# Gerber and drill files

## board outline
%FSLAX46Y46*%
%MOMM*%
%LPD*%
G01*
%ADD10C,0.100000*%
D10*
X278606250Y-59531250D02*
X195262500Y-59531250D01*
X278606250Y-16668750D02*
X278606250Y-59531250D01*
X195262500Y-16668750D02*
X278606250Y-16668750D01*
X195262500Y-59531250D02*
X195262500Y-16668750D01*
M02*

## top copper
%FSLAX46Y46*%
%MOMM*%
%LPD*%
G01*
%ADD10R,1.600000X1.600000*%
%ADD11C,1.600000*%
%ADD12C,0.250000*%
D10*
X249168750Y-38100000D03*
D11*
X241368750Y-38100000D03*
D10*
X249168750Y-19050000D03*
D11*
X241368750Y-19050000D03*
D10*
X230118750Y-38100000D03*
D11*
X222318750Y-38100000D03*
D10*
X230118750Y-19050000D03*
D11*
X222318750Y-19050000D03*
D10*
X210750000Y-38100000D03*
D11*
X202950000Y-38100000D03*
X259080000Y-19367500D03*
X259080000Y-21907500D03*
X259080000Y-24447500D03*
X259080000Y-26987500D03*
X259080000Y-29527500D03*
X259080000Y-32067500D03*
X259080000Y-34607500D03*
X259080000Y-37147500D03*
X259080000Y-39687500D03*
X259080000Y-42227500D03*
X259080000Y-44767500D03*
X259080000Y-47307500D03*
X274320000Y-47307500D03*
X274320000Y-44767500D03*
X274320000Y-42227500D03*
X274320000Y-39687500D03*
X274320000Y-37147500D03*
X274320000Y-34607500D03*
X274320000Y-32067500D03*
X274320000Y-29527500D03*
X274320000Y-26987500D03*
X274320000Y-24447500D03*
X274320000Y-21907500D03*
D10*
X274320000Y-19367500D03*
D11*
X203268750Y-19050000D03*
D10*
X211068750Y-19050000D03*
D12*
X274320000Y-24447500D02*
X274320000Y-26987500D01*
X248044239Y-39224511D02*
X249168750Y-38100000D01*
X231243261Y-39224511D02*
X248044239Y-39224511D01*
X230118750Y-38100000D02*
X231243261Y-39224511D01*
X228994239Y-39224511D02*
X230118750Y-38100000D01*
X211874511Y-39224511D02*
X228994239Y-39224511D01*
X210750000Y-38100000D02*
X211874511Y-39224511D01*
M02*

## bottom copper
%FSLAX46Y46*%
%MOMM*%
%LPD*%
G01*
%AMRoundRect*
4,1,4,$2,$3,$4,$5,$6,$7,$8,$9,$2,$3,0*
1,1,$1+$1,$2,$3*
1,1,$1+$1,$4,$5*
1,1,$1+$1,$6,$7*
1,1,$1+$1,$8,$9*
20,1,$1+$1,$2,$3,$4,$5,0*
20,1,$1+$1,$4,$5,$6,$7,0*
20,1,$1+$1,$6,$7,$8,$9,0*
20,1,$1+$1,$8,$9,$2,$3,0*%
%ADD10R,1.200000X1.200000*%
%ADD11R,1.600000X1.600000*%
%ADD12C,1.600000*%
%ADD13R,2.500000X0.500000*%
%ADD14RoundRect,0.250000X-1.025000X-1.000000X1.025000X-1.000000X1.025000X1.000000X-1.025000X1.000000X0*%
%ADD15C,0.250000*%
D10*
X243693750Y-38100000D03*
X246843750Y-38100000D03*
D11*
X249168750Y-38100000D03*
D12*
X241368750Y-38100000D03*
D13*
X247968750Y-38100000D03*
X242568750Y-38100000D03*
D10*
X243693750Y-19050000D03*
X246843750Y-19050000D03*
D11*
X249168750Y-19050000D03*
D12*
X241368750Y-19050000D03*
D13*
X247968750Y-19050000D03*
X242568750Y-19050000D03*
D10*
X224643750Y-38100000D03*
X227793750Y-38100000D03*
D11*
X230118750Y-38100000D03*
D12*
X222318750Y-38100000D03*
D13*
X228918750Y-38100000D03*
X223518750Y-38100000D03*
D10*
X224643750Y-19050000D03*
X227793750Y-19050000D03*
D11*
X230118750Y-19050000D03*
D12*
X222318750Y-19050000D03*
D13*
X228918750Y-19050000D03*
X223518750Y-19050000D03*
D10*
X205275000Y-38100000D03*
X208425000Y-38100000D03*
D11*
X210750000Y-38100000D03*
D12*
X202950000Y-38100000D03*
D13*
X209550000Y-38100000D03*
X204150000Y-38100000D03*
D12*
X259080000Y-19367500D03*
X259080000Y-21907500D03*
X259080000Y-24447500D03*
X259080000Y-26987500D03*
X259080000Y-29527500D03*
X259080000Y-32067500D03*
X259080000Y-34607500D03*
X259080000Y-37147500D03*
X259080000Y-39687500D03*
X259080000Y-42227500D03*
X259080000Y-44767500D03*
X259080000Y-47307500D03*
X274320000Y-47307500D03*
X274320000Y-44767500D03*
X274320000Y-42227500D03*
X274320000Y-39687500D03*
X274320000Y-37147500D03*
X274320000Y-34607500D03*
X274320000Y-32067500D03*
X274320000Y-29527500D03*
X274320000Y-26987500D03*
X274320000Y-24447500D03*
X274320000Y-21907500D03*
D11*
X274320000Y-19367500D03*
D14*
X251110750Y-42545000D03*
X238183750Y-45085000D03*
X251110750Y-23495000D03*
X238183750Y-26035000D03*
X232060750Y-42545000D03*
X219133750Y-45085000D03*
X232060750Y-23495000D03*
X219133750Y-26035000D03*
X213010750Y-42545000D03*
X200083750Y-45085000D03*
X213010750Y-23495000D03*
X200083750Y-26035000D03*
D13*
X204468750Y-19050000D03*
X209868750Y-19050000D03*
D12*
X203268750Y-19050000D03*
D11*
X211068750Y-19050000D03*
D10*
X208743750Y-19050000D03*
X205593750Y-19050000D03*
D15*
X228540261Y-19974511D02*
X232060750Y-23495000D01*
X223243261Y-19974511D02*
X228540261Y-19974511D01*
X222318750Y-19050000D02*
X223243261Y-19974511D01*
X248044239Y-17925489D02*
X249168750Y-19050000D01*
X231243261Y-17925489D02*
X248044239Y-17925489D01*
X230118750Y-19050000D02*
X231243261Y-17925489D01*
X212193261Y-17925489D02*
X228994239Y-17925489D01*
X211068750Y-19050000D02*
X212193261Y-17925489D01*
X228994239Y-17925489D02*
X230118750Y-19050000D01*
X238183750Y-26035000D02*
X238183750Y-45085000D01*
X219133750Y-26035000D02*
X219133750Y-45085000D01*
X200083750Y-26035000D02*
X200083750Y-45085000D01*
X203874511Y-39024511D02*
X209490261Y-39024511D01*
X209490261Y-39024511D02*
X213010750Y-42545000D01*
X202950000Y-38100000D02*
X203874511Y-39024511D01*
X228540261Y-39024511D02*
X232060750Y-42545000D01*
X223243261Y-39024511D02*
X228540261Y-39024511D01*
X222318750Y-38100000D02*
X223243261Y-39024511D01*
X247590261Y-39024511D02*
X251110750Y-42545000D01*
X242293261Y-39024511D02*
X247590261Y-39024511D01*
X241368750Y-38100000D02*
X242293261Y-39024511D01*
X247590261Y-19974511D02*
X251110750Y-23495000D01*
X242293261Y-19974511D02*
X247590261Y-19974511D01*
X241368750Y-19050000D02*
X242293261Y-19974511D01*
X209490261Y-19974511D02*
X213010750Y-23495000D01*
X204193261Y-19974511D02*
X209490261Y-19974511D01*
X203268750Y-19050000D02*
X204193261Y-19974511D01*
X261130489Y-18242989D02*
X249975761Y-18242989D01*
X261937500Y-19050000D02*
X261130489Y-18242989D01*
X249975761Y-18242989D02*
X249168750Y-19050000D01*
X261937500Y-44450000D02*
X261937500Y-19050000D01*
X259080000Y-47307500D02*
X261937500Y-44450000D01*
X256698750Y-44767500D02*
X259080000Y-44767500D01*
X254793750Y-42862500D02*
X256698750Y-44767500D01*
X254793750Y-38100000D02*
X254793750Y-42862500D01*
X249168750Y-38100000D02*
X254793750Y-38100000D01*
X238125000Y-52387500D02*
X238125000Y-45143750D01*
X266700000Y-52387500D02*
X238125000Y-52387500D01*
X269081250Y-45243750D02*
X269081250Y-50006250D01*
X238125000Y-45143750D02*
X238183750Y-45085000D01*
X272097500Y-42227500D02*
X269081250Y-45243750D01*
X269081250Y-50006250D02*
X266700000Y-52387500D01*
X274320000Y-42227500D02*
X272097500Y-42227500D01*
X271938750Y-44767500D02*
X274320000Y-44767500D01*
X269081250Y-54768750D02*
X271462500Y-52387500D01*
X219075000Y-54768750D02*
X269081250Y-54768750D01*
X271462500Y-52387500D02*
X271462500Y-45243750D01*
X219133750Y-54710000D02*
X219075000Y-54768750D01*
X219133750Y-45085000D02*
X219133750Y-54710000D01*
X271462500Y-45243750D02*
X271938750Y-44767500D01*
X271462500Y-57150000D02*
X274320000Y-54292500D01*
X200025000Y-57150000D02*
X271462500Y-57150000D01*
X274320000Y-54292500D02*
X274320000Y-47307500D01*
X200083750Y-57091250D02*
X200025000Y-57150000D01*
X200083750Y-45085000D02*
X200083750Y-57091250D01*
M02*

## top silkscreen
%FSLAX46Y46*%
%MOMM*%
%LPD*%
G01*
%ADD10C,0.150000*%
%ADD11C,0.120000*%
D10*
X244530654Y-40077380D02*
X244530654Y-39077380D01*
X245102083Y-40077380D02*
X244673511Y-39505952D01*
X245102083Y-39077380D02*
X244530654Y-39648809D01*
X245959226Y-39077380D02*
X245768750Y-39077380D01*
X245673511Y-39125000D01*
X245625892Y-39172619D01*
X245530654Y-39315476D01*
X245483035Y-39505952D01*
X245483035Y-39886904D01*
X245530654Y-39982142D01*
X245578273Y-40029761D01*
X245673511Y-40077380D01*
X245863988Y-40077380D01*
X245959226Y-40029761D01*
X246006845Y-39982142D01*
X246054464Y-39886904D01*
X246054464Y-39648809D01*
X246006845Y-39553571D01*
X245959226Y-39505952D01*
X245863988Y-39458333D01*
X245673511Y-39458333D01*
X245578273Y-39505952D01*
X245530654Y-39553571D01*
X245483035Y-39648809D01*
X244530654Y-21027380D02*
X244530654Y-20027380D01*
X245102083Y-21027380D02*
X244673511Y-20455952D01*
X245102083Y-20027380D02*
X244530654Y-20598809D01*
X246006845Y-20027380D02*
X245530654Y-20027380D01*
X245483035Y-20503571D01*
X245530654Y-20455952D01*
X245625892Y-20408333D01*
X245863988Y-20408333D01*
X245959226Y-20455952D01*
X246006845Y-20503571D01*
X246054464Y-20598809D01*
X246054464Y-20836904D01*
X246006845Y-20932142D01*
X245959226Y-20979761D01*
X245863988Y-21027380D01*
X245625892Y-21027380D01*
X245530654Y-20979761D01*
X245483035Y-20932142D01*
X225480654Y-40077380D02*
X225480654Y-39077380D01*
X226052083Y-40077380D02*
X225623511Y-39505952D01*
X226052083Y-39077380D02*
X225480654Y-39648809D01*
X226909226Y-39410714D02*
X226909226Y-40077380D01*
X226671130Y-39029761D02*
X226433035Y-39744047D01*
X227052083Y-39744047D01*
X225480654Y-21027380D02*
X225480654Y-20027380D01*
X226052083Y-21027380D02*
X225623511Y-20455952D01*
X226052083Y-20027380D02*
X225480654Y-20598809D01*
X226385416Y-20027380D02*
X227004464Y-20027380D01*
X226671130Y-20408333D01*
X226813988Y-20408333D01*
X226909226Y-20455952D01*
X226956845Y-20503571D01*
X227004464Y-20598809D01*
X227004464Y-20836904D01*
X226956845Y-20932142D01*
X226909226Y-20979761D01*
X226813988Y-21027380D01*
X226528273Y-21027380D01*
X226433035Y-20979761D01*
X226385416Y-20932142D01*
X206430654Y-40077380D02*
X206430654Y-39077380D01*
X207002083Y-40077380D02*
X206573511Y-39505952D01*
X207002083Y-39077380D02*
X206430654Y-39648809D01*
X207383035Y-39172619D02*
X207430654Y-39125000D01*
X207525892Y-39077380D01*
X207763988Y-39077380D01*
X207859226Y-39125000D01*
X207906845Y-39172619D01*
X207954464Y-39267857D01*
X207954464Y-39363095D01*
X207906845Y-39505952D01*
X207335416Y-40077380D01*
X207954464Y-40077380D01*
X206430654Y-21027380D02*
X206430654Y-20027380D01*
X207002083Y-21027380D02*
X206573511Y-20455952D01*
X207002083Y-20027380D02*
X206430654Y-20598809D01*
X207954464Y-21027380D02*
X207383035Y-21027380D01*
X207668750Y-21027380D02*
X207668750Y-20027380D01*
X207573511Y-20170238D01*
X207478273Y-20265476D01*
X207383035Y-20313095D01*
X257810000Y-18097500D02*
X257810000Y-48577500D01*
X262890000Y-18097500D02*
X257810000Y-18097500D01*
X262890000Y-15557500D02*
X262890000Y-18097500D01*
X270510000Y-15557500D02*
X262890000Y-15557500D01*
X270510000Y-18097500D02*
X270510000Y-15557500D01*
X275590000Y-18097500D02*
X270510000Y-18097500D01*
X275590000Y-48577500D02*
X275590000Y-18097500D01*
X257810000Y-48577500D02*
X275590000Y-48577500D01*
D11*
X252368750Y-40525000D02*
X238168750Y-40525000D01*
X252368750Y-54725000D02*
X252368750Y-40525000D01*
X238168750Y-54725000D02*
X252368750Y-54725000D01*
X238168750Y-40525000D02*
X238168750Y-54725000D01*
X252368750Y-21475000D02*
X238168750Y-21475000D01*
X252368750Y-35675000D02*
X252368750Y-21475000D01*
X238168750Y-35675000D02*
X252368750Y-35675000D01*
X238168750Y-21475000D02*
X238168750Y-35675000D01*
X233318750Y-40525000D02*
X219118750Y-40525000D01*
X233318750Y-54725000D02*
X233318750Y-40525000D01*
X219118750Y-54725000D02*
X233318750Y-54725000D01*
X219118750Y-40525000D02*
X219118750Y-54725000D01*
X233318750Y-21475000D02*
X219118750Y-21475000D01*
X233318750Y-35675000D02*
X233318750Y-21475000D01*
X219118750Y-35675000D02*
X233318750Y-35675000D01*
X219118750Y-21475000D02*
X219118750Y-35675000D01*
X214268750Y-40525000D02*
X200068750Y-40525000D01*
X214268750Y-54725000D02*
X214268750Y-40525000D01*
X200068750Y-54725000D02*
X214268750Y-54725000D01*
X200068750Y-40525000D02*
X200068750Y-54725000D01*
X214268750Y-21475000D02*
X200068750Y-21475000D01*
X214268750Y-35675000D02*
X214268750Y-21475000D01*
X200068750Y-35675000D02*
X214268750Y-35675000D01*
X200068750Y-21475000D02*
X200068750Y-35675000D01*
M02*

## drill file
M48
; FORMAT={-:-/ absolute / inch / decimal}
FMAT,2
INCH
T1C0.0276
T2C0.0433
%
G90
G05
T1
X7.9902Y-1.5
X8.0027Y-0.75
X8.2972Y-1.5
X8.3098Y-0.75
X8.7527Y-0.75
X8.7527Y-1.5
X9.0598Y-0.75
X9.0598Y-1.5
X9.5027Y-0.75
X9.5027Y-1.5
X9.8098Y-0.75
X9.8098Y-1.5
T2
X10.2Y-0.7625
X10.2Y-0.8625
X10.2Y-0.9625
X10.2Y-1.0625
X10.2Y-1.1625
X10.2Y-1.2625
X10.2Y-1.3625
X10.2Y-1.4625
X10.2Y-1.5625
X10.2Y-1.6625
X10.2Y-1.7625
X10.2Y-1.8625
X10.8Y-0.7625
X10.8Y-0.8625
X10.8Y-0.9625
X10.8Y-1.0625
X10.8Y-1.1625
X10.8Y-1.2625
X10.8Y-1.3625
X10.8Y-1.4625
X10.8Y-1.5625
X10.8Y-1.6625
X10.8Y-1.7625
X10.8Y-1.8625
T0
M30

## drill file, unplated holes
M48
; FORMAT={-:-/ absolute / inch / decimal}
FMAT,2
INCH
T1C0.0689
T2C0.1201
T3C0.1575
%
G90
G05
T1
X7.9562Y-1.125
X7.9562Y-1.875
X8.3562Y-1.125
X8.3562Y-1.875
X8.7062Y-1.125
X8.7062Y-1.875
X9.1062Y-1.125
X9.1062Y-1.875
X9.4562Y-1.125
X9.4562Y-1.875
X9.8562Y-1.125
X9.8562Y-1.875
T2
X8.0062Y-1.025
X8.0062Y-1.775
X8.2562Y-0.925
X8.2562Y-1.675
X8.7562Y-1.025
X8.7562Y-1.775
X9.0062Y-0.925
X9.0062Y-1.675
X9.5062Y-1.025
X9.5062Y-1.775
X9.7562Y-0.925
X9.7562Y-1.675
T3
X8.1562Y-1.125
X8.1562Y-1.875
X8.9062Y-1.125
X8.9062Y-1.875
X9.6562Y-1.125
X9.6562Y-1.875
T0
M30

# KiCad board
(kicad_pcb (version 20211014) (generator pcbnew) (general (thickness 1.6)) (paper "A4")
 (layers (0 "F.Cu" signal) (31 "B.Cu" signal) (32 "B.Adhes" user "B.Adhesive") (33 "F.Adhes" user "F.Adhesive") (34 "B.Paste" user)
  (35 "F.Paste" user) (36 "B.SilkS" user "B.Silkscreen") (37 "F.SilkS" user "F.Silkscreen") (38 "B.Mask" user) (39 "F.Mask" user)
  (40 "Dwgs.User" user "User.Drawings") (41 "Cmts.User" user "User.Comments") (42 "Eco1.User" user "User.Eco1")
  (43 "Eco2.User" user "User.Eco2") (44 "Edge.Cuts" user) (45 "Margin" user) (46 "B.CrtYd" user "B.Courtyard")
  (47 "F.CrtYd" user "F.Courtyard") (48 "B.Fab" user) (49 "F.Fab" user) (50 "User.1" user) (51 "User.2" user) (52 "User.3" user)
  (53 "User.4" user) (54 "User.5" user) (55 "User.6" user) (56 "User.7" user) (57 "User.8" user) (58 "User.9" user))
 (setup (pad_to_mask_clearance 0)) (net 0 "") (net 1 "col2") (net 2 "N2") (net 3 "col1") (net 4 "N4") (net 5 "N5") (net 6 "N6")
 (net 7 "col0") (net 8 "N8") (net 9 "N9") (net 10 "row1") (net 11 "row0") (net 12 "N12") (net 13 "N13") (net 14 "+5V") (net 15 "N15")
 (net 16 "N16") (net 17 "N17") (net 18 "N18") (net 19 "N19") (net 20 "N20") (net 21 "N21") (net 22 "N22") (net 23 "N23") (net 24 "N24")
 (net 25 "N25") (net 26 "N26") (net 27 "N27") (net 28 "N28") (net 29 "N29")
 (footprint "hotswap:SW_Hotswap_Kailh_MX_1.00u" (layer "F.Cu") (at 245.26875 28.575)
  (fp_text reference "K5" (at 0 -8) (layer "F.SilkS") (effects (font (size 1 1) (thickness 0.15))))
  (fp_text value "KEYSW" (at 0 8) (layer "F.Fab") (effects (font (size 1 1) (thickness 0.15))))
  (fp_line (start -7.1 7.1) (end 7.1 7.1) (layer "F.SilkS") (width 0.12))
  (fp_line (start -7.1 -7.1) (end -7.1 7.1) (layer "F.SilkS") (width 0.12))
  (fp_line (start 7.1 -7.1) (end -7.1 -7.1) (layer "F.SilkS") (width 0.12))
  (fp_line (start 7.1 7.1) (end 7.1 -7.1) (layer "F.SilkS") (width 0.12))
  (pad "" np_thru_hole circle locked (at 0 0) (size 4 4) (drill 4) (layers *.Cu *.Mask))
  (pad "" np_thru_hole circle locked (at 2.54 -5.08) (size 3.05 3.05) (drill 3.05) (layers *.Cu *.Mask))
  (pad "" np_thru_hole circle locked (at -3.81 -2.54) (size 3.05 3.05) (drill 3.05) (layers *.Cu *.Mask))
  (pad "" np_thru_hole circle locked (at -5.08 0) (size 1.75 1.75) (drill 1.75) (layers *.Cu *.Mask))
  (pad "" np_thru_hole circle locked (at 5.08 0) (size 1.75 1.75) (drill 1.75) (layers *.Cu *.Mask))
  (pad "1" smd roundrect locked (at -7.085 -2.54) (size 2.55 2.5) (layers "B.Cu" "B.Paste" "B.Mask") (roundrect_rratio 0.1) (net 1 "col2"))
  (pad "2" smd roundrect locked (at 5.842 -5.08) (size 2.55 2.5) (layers "B.Cu" "B.Paste" "B.Mask") (roundrect_rratio 0.1) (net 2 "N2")))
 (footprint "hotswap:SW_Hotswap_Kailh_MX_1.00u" (layer "F.Cu") (at 226.21875 47.625)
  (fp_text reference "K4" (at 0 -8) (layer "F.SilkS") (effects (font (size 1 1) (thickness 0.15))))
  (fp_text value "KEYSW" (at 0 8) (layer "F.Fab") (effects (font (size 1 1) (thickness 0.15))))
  (fp_line (start -7.1 -7.1) (end -7.1 7.1) (layer "F.SilkS") (width 0.12))
  (fp_line (start -7.1 7.1) (end 7.1 7.1) (layer "F.SilkS") (width 0.12))
  (fp_line (start 7.1 -7.1) (end -7.1 -7.1) (layer "F.SilkS") (width 0.12))
  (fp_line (start 7.1 7.1) (end 7.1 -7.1) (layer "F.SilkS") (width 0.12))
  (pad "" np_thru_hole circle locked (at 2.54 -5.08) (size 3.05 3.05) (drill 3.05) (layers *.Cu *.Mask))
  (pad "" np_thru_hole circle locked (at 5.08 0) (size 1.75 1.75) (drill 1.75) (layers *.Cu *.Mask))
  (pad "" np_thru_hole circle locked (at -5.08 0) (size 1.75 1.75) (drill 1.75) (layers *.Cu *.Mask))
  (pad "" np_thru_hole circle locked (at -3.81 -2.54) (size 3.05 3.05) (drill 3.05) (layers *.Cu *.Mask))
  (pad "" np_thru_hole circle locked (at 0 0) (size 4 4) (drill 4) (layers *.Cu *.Mask))
  (pad "1" smd roundrect locked (at -7.085 -2.54) (size 2.55 2.5) (layers "B.Cu" "B.Paste" "B.Mask") (roundrect_rratio 0.1) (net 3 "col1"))
  (pad "2" smd roundrect locked (at 5.842 -5.08) (size 2.55 2.5) (layers "B.Cu" "B.Paste" "B.Mask") (roundrect_rratio 0.1) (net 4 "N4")))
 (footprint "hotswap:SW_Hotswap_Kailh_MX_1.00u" (layer "F.Cu") (at 226.21875 28.575)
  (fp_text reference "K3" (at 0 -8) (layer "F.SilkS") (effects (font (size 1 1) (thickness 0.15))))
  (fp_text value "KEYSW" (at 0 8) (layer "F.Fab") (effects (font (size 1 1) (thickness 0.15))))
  (fp_line (start 7.1 7.1) (end 7.1 -7.1) (layer "F.SilkS") (width 0.12))
  (fp_line (start -7.1 -7.1) (end -7.1 7.1) (layer "F.SilkS") (width 0.12))
  (fp_line (start -7.1 7.1) (end 7.1 7.1) (layer "F.SilkS") (width 0.12))
  (fp_line (start 7.1 -7.1) (end -7.1 -7.1) (layer "F.SilkS") (width 0.12))
  (pad "" np_thru_hole circle locked (at 5.08 0) (size 1.75 1.75) (drill 1.75) (layers *.Cu *.Mask))
  (pad "" np_thru_hole circle locked (at -5.08 0) (size 1.75 1.75) (drill 1.75) (layers *.Cu *.Mask))
  (pad "" np_thru_hole circle locked (at 0 0) (size 4 4) (drill 4) (layers *.Cu *.Mask))
  (pad "" np_thru_hole circle locked (at -3.81 -2.54) (size 3.05 3.05) (drill 3.05) (layers *.Cu *.Mask))
  (pad "" np_thru_hole circle locked (at 2.54 -5.08) (size 3.05 3.05) (drill 3.05) (layers *.Cu *.Mask))
  (pad "1" smd roundrect locked (at -7.085 -2.54) (size 2.55 2.5) (layers "B.Cu" "B.Paste" "B.Mask") (roundrect_rratio 0.1) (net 3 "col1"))
  (pad "2" smd roundrect locked (at 5.842 -5.08) (size 2.55 2.5) (layers "B.Cu" "B.Paste" "B.Mask") (roundrect_rratio 0.1) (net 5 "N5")))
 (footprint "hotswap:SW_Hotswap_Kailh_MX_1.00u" (layer "F.Cu") (at 245.26875 47.625)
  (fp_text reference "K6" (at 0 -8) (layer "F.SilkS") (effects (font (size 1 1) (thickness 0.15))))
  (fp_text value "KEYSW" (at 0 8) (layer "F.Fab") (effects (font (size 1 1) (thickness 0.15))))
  (fp_line (start -7.1 -7.1) (end -7.1 7.1) (layer "F.SilkS") (width 0.12))
  (fp_line (start 7.1 7.1) (end 7.1 -7.1) (layer "F.SilkS") (width 0.12))
  (fp_line (start -7.1 7.1) (end 7.1 7.1) (layer "F.SilkS") (width 0.12))
  (fp_line (start 7.1 -7.1) (end -7.1 -7.1) (layer "F.SilkS") (width 0.12))
  (pad "" np_thru_hole circle locked (at 0 0) (size 4 4) (drill 4) (layers *.Cu *.Mask))
  (pad "" np_thru_hole circle locked (at -5.08 0) (size 1.75 1.75) (drill 1.75) (layers *.Cu *.Mask))
  (pad "" np_thru_hole circle locked (at -3.81 -2.54) (size 3.05 3.05) (drill 3.05) (layers *.Cu *.Mask))
  (pad "" np_thru_hole circle locked (at 5.08 0) (size 1.75 1.75) (drill 1.75) (layers *.Cu *.Mask))
  (pad "" np_thru_hole circle locked (at 2.54 -5.08) (size 3.05 3.05) (drill 3.05) (layers *.Cu *.Mask))
  (pad "1" smd roundrect locked (at -7.085 -2.54) (size 2.55 2.5) (layers "B.Cu" "B.Paste" "B.Mask") (roundrect_rratio 0.1) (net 1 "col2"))
  (pad "2" smd roundrect locked (at 5.842 -5.08) (size 2.55 2.5) (layers "B.Cu" "B.Paste" "B.Mask") (roundrect_rratio 0.1) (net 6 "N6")))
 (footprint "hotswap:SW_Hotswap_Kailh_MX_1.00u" (layer "F.Cu") (at 207.16875 28.575)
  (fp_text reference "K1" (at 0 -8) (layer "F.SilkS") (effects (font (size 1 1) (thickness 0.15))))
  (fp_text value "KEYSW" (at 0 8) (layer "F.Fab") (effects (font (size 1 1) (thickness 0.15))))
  (fp_line (start -7.1 -7.1) (end -7.1 7.1) (layer "F.SilkS") (width 0.12))
  (fp_line (start 7.1 7.1) (end 7.1 -7.1) (layer "F.SilkS") (width 0.12))
  (fp_line (start -7.1 7.1) (end 7.1 7.1) (layer "F.SilkS") (width 0.12))
  (fp_line (start 7.1 -7.1) (end -7.1 -7.1) (layer "F.SilkS") (width 0.12))
  (pad "" np_thru_hole circle locked (at 2.54 -5.08) (size 3.05 3.05) (drill 3.05) (layers *.Cu *.Mask))
  (pad "" np_thru_hole circle locked (at 5.08 0) (size 1.75 1.75) (drill 1.75) (layers *.Cu *.Mask))
  (pad "" np_thru_hole circle locked (at -5.08 0) (size 1.75 1.75) (drill 1.75) (layers *.Cu *.Mask))
  (pad "" np_thru_hole circle locked (at 0 0) (size 4 4) (drill 4) (layers *.Cu *.Mask))
  (pad "" np_thru_hole circle locked (at -3.81 -2.54) (size 3.05 3.05) (drill 3.05) (layers *.Cu *.Mask))
  (pad "1" smd roundrect locked (at -7.085 -2.54) (size 2.55 2.5) (layers "B.Cu" "B.Paste" "B.Mask") (roundrect_rratio 0.1) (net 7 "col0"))
  (pad "2" smd roundrect locked (at 5.842 -5.08) (size 2.55 2.5) (layers "B.Cu" "B.Paste" "B.Mask") (roundrect_rratio 0.1) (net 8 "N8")))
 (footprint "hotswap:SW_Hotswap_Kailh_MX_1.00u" (layer "F.Cu") (at 207.16875 47.625)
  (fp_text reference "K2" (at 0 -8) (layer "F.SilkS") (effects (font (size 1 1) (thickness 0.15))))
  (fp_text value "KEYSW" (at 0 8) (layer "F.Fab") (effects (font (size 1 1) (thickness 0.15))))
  (fp_line (start 7.1 -7.1) (end -7.1 -7.1) (layer "F.SilkS") (width 0.12))
  (fp_line (start 7.1 7.1) (end 7.1 -7.1) (layer "F.SilkS") (width 0.12))
  (fp_line (start -7.1 -7.1) (end -7.1 7.1) (layer "F.SilkS") (width 0.12))
  (fp_line (start -7.1 7.1) (end 7.1 7.1) (layer "F.SilkS") (width 0.12))
  (pad "" np_thru_hole circle locked (at 2.54 -5.08) (size 3.05 3.05) (drill 3.05) (layers *.Cu *.Mask))
  (pad "" np_thru_hole circle locked (at -5.08 0) (size 1.75 1.75) (drill 1.75) (layers *.Cu *.Mask))
  (pad "" np_thru_hole circle locked (at -3.81 -2.54) (size 3.05 3.05) (drill 3.05) (layers *.Cu *.Mask))
  (pad "" np_thru_hole circle locked (at 0 0) (size 4 4) (drill 4) (layers *.Cu *.Mask))
  (pad "" np_thru_hole circle locked (at 5.08 0) (size 1.75 1.75) (drill 1.75) (layers *.Cu *.Mask))
  (pad "1" smd roundrect locked (at -7.085 -2.54) (size 2.55 2.5) (layers "B.Cu" "B.Paste" "B.Mask") (roundrect_rratio 0.1) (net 7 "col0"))
  (pad "2" smd roundrect locked (at 5.842 -5.08) (size 2.55 2.5) (layers "B.Cu" "B.Paste" "B.Mask") (roundrect_rratio 0.1) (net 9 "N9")))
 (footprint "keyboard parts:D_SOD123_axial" (layer "B.Cu") (at 226.21875 38.1 180)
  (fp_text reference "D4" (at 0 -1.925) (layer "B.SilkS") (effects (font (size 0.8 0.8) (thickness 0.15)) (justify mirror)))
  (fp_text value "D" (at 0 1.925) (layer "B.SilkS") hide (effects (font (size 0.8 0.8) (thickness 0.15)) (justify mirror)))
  (pad "1" smd rect locked (at -2.7 0 180) (size 2.5 0.5) (layers "B.Cu") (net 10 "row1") (solder_mask_margin -999))
  (pad "1" smd rect locked (at -1.575 0 180) (size 1.2 1.2) (layers "B.Cu" "B.Paste" "B.Mask") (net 10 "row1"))
  (pad "1" thru_hole rect locked (at -3.9 0 180) (size 1.6 1.6) (drill 0.7) (layers *.Cu *.Mask "B.SilkS") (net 10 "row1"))
  (pad "2" thru_hole circle locked (at 3.9 0 180) (size 1.6 1.6) (drill 0.7) (layers *.Cu *.Mask "B.SilkS") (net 4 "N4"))
  (pad "2" smd rect locked (at 2.7 0 180) (size 2.5 0.5) (layers "B.Cu") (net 4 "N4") (solder_mask_margin -999))
  (pad "2" smd rect locked (at 1.575 0 180) (size 1.2 1.2) (layers "B.Cu" "B.Paste" "B.Mask") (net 4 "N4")))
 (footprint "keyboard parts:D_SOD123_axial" (layer "B.Cu") (at 245.26875 19.05 180)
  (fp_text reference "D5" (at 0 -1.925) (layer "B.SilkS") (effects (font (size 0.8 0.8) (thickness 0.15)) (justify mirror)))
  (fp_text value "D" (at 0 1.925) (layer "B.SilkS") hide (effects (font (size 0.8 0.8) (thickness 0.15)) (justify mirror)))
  (pad "1" thru_hole rect locked (at -3.9 0 180) (size 1.6 1.6) (drill 0.7) (layers *.Cu *.Mask "B.SilkS") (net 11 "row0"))
  (pad "1" smd rect locked (at -2.7 0 180) (size 2.5 0.5) (layers "B.Cu") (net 11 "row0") (solder_mask_margin -999))
  (pad "1" smd rect locked (at -1.575 0 180) (size 1.2 1.2) (layers "B.Cu" "B.Paste" "B.Mask") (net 11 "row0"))
  (pad "2" smd rect locked (at 2.7 0 180) (size 2.5 0.5) (layers "B.Cu") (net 2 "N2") (solder_mask_margin -999))
  (pad "2" smd rect locked (at 1.575 0 180) (size 1.2 1.2) (layers "B.Cu" "B.Paste" "B.Mask") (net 2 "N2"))
  (pad "2" thru_hole circle locked (at 3.9 0 180) (size 1.6 1.6) (drill 0.7) (layers *.Cu *.Mask "B.SilkS") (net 2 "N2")))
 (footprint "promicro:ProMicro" (layer "B.Cu") (at 266.7 33.3375 -90)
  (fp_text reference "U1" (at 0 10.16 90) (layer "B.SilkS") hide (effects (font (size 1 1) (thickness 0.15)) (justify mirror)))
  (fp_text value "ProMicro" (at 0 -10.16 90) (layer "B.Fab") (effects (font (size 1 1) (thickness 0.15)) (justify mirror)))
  (fp_line (start -15.24 -8.89) (end -15.24 -3.81) (layer "F.SilkS") (width 0.15))
  (fp_line (start -15.24 -3.81) (end -17.78 -3.81) (layer "F.SilkS") (width 0.15))
  (fp_line (start 15.24 8.89) (end 15.24 -8.89) (layer "F.SilkS") (width 0.15))
  (fp_line (start -15.24 8.89) (end 15.24 8.89) (layer "F.SilkS") (width 0.15))
  (fp_line (start -17.78 3.81) (end -15.24 3.81) (layer "F.SilkS") (width 0.15))
  (fp_line (start 15.24 -8.89) (end -15.24 -8.89) (layer "F.SilkS") (width 0.15))
  (fp_line (start -17.78 -3.81) (end -17.78 3.81) (layer "F.SilkS") (width 0.15))
  (fp_line (start -15.24 3.81) (end -15.24 8.89) (layer "F.SilkS") (width 0.15))
  (pad "1" thru_hole rect locked (at -13.97 -7.62 270) (size 1.6 1.6) (drill 1.1) (layers *.Cu *.Mask "B.SilkS") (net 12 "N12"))
  (pad "2" thru_hole circle locked (at -11.43 -7.62 270) (size 1.6 1.6) (drill 1.1) (layers *.Cu *.Mask "B.SilkS") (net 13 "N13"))
  (pad "3" thru_hole circle locked (at -8.89 -7.62 270) (size 1.6 1.6) (drill 1.1) (layers *.Cu *.Mask "B.SilkS") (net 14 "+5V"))
  (pad "4" thru_hole circle locked (at -6.35 -7.62 270) (size 1.6 1.6) (drill 1.1) (layers *.Cu *.Mask "B.SilkS") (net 14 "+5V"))
  (pad "5" thru_hole circle locked (at -3.81 -7.62 270) (size 1.6 1.6) (drill 1.1) (layers *.Cu *.Mask "B.SilkS") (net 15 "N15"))
  (pad "6" thru_hole circle locked (at -1.27 -7.62 270) (size 1.6 1.6) (drill 1.1) (layers *.Cu *.Mask "B.SilkS") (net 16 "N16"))
  (pad "7" thru_hole circle locked (at 1.27 -7.62 270) (size 1.6 1.6) (drill 1.1) (layers *.Cu *.Mask "B.SilkS") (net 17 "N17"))
  (pad "8" thru_hole circle locked (at 3.81 -7.62 270) (size 1.6 1.6) (drill 1.1) (layers *.Cu *.Mask "B.SilkS") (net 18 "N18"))
  (pad "9" thru_hole circle locked (at 6.35 -7.62 270) (size 1.6 1.6) (drill 1.1) (layers *.Cu *.Mask "B.SilkS") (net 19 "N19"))
  (pad "10" thru_hole circle locked (at 8.89 -7.62 270) (size 1.6 1.6) (drill 1.1) (layers *.Cu *.Mask "B.SilkS") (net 1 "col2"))
  (pad "11" thru_hole circle locked (at 11.43 -7.62 270) (size 1.6 1.6) (drill 1.1) (layers *.Cu *.Mask "B.SilkS") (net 3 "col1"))
  (pad "12" thru_hole circle locked (at 13.97 -7.62 270) (size 1.6 1.6) (drill 1.1) (layers *.Cu *.Mask "B.SilkS") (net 7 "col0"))
  (pad "13" thru_hole circle locked (at 13.97 7.62 270) (size 1.6 1.6) (drill 1.1) (layers *.Cu *.Mask "B.SilkS") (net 11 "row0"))
  (pad "14" thru_hole circle locked (at 11.43 7.62 270) (size 1.6 1.6) (drill 1.1) (layers *.Cu *.Mask "B.SilkS") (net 10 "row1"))
  (pad "15" thru_hole circle locked (at 8.89 7.62 270) (size 1.6 1.6) (drill 1.1) (layers *.Cu *.Mask "B.SilkS") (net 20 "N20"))
  (pad "16" thru_hole circle locked (at 6.35 7.62 270) (size 1.6 1.6) (drill 1.1) (layers *.Cu *.Mask "B.SilkS") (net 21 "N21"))
  (pad "17" thru_hole circle locked (at 3.81 7.62 270) (size 1.6 1.6) (drill 1.1) (layers *.Cu *.Mask "B.SilkS") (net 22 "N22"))
  (pad "18" thru_hole circle locked (at 1.27 7.62 270) (size 1.6 1.6) (drill 1.1) (layers *.Cu *.Mask "B.SilkS") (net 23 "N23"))
  (pad "19" thru_hole circle locked (at -1.27 7.62 270) (size 1.6 1.6) (drill 1.1) (layers *.Cu *.Mask "B.SilkS") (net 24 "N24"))
  (pad "20" thru_hole circle locked (at -3.81 7.62 270) (size 1.6 1.6) (drill 1.1) (layers *.Cu *.Mask "B.SilkS") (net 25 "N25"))
  (pad "21" thru_hole circle locked (at -6.35 7.62 270) (size 1.6 1.6) (drill 1.1) (layers *.Cu *.Mask "B.SilkS") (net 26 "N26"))
  (pad "22" thru_hole circle locked (at -8.89 7.62 270) (size 1.6 1.6) (drill 1.1) (layers *.Cu *.Mask "B.SilkS") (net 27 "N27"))
  (pad "23" thru_hole circle locked (at -11.43 7.62 270) (size 1.6 1.6) (drill 1.1) (layers *.Cu *.Mask "B.SilkS") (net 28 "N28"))
  (pad "24" thru_hole circle locked (at -13.97 7.62 270) (size 1.6 1.6) (drill 1.1) (layers *.Cu *.Mask "B.SilkS") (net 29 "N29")))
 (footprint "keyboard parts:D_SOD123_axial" (layer "B.Cu") (at 245.26875 38.1 180)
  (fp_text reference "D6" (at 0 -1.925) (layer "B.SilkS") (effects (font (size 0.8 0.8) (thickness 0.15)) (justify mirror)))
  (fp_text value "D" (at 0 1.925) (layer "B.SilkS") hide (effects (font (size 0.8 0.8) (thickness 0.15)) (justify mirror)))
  (pad "1" smd rect locked (at -1.575 0 180) (size 1.2 1.2) (layers "B.Cu" "B.Paste" "B.Mask") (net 10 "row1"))
  (pad "1" thru_hole rect locked (at -3.9 0 180) (size 1.6 1.6) (drill 0.7) (layers *.Cu *.Mask "B.SilkS") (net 10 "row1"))
  (pad "1" smd rect locked (at -2.7 0 180) (size 2.5 0.5) (layers "B.Cu") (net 10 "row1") (solder_mask_margin -999))
  (pad "2" smd rect locked (at 1.575 0 180) (size 1.2 1.2) (layers "B.Cu" "B.Paste" "B.Mask") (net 6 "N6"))
  (pad "2" smd rect locked (at 2.7 0 180) (size 2.5 0.5) (layers "B.Cu") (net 6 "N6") (solder_mask_margin -999))
  (pad "2" thru_hole circle locked (at 3.9 0 180) (size 1.6 1.6) (drill 0.7) (layers *.Cu *.Mask "B.SilkS") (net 6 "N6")))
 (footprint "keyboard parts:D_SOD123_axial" (layer "B.Cu") (at 226.21875 19.05 180)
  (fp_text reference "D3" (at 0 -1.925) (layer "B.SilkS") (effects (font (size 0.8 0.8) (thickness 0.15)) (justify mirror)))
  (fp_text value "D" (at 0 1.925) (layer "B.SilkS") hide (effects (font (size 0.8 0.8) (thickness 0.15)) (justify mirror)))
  (pad "1" smd rect locked (at -2.7 0 180) (size 2.5 0.5) (layers "B.Cu") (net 11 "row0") (solder_mask_margin -999))
  (pad "1" smd rect locked (at -1.575 0 180) (size 1.2 1.2) (layers "B.Cu" "B.Paste" "B.Mask") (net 11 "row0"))
  (pad "1" thru_hole rect locked (at -3.9 0 180) (size 1.6 1.6) (drill 0.7) (layers *.Cu *.Mask "B.SilkS") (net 11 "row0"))
  (pad "2" thru_hole circle locked (at 3.9 0 180) (size 1.6 1.6) (drill 0.7) (layers *.Cu *.Mask "B.SilkS") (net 5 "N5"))
  (pad "2" smd rect locked (at 2.7 0 180) (size 2.5 0.5) (layers "B.Cu") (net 5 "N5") (solder_mask_margin -999))
  (pad "2" smd rect locked (at 1.575 0 180) (size 1.2 1.2) (layers "B.Cu" "B.Paste" "B.Mask") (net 5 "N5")))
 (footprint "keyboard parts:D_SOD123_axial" (layer "B.Cu") (at 207.16875 19.05 180)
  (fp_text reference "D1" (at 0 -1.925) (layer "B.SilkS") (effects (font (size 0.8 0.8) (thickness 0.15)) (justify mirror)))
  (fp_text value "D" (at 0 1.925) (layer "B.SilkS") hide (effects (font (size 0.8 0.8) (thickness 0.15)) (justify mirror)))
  (pad "1" smd rect locked (at -1.575 0 180) (size 1.2 1.2) (layers "B.Cu" "B.Paste" "B.Mask") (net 11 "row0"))
  (pad "1" smd rect locked (at -2.7 0 180) (size 2.5 0.5) (layers "B.Cu") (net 11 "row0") (solder_mask_margin -999))
  (pad "1" thru_hole rect locked (at -3.9 0 180) (size 1.6 1.6) (drill 0.7) (layers *.Cu *.Mask "B.SilkS") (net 11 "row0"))
  (pad "2" smd rect locked (at 2.7 0 180) (size 2.5 0.5) (layers "B.Cu") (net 8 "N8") (solder_mask_margin -999))
  (pad "2" thru_hole circle locked (at 3.9 0 180) (size 1.6 1.6) (drill 0.7) (layers *.Cu *.Mask "B.SilkS") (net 8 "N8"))
  (pad "2" smd rect locked (at 1.575 0 180) (size 1.2 1.2) (layers "B.Cu" "B.Paste" "B.Mask") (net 8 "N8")))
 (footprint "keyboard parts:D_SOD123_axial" (layer "B.Cu") (at 206.85 38.1 180)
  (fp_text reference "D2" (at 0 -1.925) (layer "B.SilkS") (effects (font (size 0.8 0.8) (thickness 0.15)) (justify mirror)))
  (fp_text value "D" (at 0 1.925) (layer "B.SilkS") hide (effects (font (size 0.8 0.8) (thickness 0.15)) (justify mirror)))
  (pad "1" smd rect locked (at -1.575 0 180) (size 1.2 1.2) (layers "B.Cu" "B.Paste" "B.Mask") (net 10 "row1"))
  (pad "1" smd rect locked (at -2.7 0 180) (size 2.5 0.5) (layers "B.Cu") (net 10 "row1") (solder_mask_margin -999))
  (pad "1" thru_hole rect locked (at -3.9 0 180) (size 1.6 1.6) (drill 0.7) (layers *.Cu *.Mask "B.SilkS") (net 10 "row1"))
  (pad "2" smd rect locked (at 1.575 0 180) (size 1.2 1.2) (layers "B.Cu" "B.Paste" "B.Mask") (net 9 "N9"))
  (pad "2" smd rect locked (at 2.7 0 180) (size 2.5 0.5) (layers "B.Cu") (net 9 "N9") (solder_mask_margin -999))
  (pad "2" thru_hole circle locked (at 3.9 0 180) (size 1.6 1.6) (drill 0.7) (layers *.Cu *.Mask "B.SilkS") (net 9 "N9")))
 (gr_line (start 195.2625 16.66875) (end 278.60625 16.66875) (layer "Edge.Cuts") (width 0.1))
 (gr_line (start 278.60625 59.53125) (end 195.2625 59.53125) (layer "Edge.Cuts") (width 0.1))
 (gr_line (start 278.60625 16.66875) (end 278.60625 59.53125) (layer "Edge.Cuts") (width 0.1))
 (gr_line (start 195.2625 59.53125) (end 195.2625 16.66875) (layer "Edge.Cuts") (width 0.1))
 (segment (start 209.490261 19.974511) (end 213.01075 23.495) (width 0.25) (layer "B.Cu") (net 8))
 (segment (start 204.193261 19.974511) (end 209.490261 19.974511) (width 0.25) (layer "B.Cu") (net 8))
 (segment (start 203.26875 19.05) (end 204.193261 19.974511) (width 0.25) (layer "B.Cu") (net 8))
 (segment (start 202.95 38.1) (end 203.874511 39.024511) (width 0.25) (layer "B.Cu") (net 9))
 (segment (start 203.874511 39.024511) (end 209.490261 39.024511) (width 0.25) (layer "B.Cu") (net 9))
 (segment (start 209.490261 39.024511) (end 213.01075 42.545) (width 0.25) (layer "B.Cu") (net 9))
 (segment (start 222.31875 19.05) (end 223.243261 19.974511) (width 0.25) (layer "B.Cu") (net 5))
 (segment (start 223.243261 19.974511) (end 228.540261 19.974511) (width 0.25) (layer "B.Cu") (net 5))
 (segment (start 228.540261 19.974511) (end 232.06075 23.495) (width 0.25) (layer "B.Cu") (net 5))
 (segment (start 222.31875 38.1) (end 223.243261 39.024511) (width 0.25) (layer "B.Cu") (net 4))
 (segment (start 228.540261 39.024511) (end 232.06075 42.545) (width 0.25) (layer "B.Cu") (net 4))
 (segment (start 223.243261 39.024511) (end 228.540261 39.024511) (width 0.25) (layer "B.Cu") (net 4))
 (segment (start 242.293261 19.974511) (end 247.590261 19.974511) (width 0.25) (layer "B.Cu") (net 2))
 (segment (start 247.590261 19.974511) (end 251.11075 23.495) (width 0.25) (layer "B.Cu") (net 2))
 (segment (start 241.36875 19.05) (end 242.293261 19.974511) (width 0.25) (layer "B.Cu") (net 2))
 (segment (start 261.9375 19.05) (end 261.130489 18.242989) (width 0.25) (layer "B.Cu") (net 11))
 (segment (start 228.994239 17.925489) (end 230.11875 19.05) (width 0.25) (layer "B.Cu") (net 11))
 (segment (start 261.9375 44.45) (end 261.9375 19.05) (width 0.25) (layer "B.Cu") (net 11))
 (segment (start 230.11875 19.05) (end 231.243261 17.925489) (width 0.25) (layer "B.Cu") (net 11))
 (segment (start 259.08 47.3075) (end 261.9375 44.45) (width 0.25) (layer "B.Cu") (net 11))
 (segment (start 211.06875 19.05) (end 212.193261 17.925489) (width 0.25) (layer "B.Cu") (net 11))
 (segment (start 248.044239 17.925489) (end 249.16875 19.05) (width 0.25) (layer "B.Cu") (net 11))
 (segment (start 249.975761 18.242989) (end 249.16875 19.05) (width 0.25) (layer "B.Cu") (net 11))
 (segment (start 212.193261 17.925489) (end 228.994239 17.925489) (width 0.25) (layer "B.Cu") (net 11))
 (segment (start 231.243261 17.925489) (end 248.044239 17.925489) (width 0.25) (layer "B.Cu") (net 11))
 (segment (start 261.130489 18.242989) (end 249.975761 18.242989) (width 0.25) (layer "B.Cu") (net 11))
 (segment (start 241.36875 38.1) (end 242.293261 39.024511) (width 0.25) (layer "B.Cu") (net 6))
 (segment (start 247.590261 39.024511) (end 251.11075 42.545) (width 0.25) (layer "B.Cu") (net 6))
 (segment (start 242.293261 39.024511) (end 247.590261 39.024511) (width 0.25) (layer "B.Cu") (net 6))
 (segment (start 210.75 38.1) (end 211.874511 39.224511) (width 0.25) (layer "F.Cu") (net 10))
 (segment (start 248.044239 39.224511) (end 249.16875 38.1) (width 0.25) (layer "F.Cu") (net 10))
 (segment (start 231.243261 39.224511) (end 248.044239 39.224511) (width 0.25) (layer "F.Cu") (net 10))
 (segment (start 228.994239 39.224511) (end 230.11875 38.1) (width 0.25) (layer "F.Cu") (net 10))
 (segment (start 230.11875 38.1) (end 231.243261 39.224511) (width 0.25) (layer "F.Cu") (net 10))
 (segment (start 211.874511 39.224511) (end 228.994239 39.224511) (width 0.25) (layer "F.Cu") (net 10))
 (segment (start 256.69875 44.7675) (end 259.08 44.7675) (width 0.25) (layer "B.Cu") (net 10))
 (segment (start 254.79375 38.1) (end 254.79375 42.8625) (width 0.25) (layer "B.Cu") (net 10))
 (segment (start 249.16875 38.1) (end 254.79375 38.1) (width 0.25) (layer "B.Cu") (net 10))
 (segment (start 254.79375 42.8625) (end 256.69875 44.7675) (width 0.25) (layer "B.Cu") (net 10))
 (segment (start 200.08375 45.085) (end 200.08375 57.09125) (width 0.25) (layer "B.Cu") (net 7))
 (segment (start 200.025 57.15) (end 271.4625 57.15) (width 0.25) (layer "B.Cu") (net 7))
 (segment (start 274.32 54.2925) (end 274.32 47.3075) (width 0.25) (layer "B.Cu") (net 7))
 (segment (start 271.4625 57.15) (end 274.32 54.2925) (width 0.25) (layer "B.Cu") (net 7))
 (segment (start 200.08375 57.09125) (end 200.025 57.15) (width 0.25) (layer "B.Cu") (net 7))
 (segment (start 200.08375 26.035) (end 200.08375 45.085) (width 0.25) (layer "B.Cu") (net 7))
 (segment (start 271.4625 45.24375) (end 271.93875 44.7675) (width 0.25) (layer "B.Cu") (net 3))
 (segment (start 269.08125 54.76875) (end 271.4625 52.3875) (width 0.25) (layer "B.Cu") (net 3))
 (segment (start 219.13375 54.71) (end 219.075 54.76875) (width 0.25) (layer "B.Cu") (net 3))
 (segment (start 219.13375 26.035) (end 219.13375 45.085) (width 0.25) (layer "B.Cu") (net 3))
 (segment (start 219.13375 45.085) (end 219.13375 54.71) (width 0.25) (layer "B.Cu") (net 3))
 (segment (start 271.93875 44.7675) (end 274.32 44.7675) (width 0.25) (layer "B.Cu") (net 3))
 (segment (start 271.4625 52.3875) (end 271.4625 45.24375) (width 0.25) (layer "B.Cu") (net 3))
 (segment (start 219.075 54.76875) (end 269.08125 54.76875) (width 0.25) (layer "B.Cu") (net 3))
 (segment (start 238.125 52.3875) (end 238.125 45.14375) (width 0.25) (layer "B.Cu") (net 1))
 (segment (start 274.32 42.2275) (end 272.0975 42.2275) (width 0.25) (layer "B.Cu") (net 1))
 (segment (start 272.0975 42.2275) (end 269.08125 45.24375) (width 0.25) (layer "B.Cu") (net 1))
 (segment (start 266.7 52.3875) (end 238.125 52.3875) (width 0.25) (layer "B.Cu") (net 1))
 (segment (start 238.125 45.14375) (end 238.18375 45.085) (width 0.25) (layer "B.Cu") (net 1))
 (segment (start 269.08125 45.24375) (end 269.08125 50.00625) (width 0.25) (layer "B.Cu") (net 1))
 (segment (start 238.18375 26.035) (end 238.18375 45.085) (width 0.25) (layer "B.Cu") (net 1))
 (segment (start 269.08125 50.00625) (end 266.7 52.3875) (width 0.25) (layer "B.Cu") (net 1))
 (segment (start 274.32 24.4475) (end 274.32 26.9875) (width 0.25) (layer "F.Cu") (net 14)))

